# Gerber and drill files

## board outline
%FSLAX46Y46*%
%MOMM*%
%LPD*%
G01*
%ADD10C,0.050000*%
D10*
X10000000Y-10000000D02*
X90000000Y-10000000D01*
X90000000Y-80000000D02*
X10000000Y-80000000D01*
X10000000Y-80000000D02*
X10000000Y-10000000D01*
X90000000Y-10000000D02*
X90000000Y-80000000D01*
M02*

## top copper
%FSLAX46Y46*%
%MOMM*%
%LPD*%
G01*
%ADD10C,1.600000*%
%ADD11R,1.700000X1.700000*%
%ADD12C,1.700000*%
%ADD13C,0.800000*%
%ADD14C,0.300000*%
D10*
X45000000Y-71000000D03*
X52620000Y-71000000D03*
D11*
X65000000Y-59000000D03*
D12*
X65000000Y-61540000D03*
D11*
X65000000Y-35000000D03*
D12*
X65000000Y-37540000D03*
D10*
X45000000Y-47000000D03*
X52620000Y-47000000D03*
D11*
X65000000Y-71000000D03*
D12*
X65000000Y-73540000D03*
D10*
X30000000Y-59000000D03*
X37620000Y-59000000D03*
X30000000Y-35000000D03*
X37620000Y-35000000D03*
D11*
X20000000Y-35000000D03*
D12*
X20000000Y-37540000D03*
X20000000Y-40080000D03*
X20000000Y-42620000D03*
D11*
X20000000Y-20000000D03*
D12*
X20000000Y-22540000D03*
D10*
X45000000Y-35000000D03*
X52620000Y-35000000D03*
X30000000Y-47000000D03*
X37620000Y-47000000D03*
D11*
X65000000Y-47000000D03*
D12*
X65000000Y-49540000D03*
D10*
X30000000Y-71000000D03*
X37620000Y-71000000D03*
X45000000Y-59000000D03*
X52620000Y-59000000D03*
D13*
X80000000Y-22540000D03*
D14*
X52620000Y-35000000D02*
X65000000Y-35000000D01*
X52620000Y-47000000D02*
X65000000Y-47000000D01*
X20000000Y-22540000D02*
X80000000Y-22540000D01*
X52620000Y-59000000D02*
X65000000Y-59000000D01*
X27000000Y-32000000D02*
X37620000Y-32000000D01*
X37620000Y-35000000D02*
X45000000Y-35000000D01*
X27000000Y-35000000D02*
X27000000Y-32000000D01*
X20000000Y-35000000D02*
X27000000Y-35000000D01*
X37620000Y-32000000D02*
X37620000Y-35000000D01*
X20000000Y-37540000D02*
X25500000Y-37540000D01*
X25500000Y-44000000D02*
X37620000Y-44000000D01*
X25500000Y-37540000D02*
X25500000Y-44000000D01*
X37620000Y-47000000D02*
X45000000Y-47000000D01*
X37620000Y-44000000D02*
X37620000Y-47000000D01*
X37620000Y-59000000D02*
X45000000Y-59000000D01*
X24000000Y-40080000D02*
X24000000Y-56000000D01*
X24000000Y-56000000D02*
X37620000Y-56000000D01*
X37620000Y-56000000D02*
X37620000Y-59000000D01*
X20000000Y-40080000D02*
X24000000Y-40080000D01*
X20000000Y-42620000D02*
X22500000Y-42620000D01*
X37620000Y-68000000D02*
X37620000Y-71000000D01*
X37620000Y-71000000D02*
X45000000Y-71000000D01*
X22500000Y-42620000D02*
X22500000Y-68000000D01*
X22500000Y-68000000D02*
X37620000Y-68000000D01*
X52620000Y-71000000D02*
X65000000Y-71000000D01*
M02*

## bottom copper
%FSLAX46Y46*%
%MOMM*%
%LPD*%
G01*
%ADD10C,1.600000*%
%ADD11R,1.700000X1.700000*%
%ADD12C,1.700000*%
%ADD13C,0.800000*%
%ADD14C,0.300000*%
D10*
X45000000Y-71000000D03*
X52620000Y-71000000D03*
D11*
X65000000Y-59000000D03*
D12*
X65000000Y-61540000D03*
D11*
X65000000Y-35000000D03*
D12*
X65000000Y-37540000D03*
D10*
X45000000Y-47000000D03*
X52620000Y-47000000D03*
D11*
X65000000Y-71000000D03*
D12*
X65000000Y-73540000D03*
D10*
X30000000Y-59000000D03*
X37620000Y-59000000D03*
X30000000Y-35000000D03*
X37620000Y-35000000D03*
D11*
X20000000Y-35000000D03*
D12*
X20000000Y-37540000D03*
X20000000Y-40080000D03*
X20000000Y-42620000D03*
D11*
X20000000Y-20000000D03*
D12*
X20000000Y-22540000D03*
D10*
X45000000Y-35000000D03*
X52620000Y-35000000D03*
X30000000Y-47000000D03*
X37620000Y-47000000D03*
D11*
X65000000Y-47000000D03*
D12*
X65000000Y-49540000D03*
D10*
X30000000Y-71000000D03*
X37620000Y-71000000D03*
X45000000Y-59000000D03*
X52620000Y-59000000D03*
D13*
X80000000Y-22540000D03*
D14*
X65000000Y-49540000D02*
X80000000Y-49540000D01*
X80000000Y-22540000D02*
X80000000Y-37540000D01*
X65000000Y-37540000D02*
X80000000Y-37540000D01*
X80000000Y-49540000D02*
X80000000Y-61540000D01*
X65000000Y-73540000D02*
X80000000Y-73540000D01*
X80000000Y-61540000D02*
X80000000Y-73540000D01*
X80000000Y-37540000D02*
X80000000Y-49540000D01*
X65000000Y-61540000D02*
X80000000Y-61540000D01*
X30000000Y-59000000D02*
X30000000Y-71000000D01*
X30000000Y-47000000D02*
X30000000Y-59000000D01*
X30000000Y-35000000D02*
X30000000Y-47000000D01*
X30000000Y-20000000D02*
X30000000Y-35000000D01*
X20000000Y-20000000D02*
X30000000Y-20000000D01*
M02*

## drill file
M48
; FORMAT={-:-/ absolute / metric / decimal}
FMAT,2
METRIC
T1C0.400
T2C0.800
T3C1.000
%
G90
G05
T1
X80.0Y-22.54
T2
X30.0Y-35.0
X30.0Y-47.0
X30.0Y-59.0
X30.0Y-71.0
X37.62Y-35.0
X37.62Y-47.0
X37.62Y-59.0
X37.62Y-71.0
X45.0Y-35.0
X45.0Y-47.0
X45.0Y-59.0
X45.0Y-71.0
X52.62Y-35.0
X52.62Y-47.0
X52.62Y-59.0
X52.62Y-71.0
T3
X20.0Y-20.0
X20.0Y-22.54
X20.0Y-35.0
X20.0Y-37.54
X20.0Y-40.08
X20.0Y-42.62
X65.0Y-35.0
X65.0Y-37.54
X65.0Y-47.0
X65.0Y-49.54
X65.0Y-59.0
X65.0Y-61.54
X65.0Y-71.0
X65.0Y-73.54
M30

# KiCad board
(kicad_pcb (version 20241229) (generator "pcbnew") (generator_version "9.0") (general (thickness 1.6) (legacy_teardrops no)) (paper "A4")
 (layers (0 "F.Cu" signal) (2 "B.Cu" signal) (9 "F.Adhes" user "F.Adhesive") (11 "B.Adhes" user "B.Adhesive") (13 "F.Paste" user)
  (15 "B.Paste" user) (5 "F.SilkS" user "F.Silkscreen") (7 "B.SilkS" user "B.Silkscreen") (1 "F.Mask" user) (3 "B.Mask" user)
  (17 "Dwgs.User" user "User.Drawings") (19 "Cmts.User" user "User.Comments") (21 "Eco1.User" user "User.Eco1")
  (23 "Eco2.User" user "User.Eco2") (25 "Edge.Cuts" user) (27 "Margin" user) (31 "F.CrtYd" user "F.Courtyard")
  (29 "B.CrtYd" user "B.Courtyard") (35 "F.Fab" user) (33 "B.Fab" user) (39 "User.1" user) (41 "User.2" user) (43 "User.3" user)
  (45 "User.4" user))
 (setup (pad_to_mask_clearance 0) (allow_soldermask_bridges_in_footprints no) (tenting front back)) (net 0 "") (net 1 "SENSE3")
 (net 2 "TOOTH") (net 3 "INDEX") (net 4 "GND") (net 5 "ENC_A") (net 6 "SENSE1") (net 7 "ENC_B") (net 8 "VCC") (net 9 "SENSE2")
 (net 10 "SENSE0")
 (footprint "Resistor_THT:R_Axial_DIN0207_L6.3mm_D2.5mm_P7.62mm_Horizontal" (layer "F.Cu") (at 45 71)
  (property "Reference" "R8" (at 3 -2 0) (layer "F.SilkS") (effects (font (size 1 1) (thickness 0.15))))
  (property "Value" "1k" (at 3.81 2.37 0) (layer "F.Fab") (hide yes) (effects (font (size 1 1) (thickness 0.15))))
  (pad "1" thru_hole circle (at 0 0) (size 1.6 1.6) (drill 0.8) (layers "*.Cu" "*.Mask") (remove_unused_layers no) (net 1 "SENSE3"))
  (pad "2" thru_hole circle (at 7.62 0) (size 1.6 1.6) (drill 0.8) (layers "*.Cu" "*.Mask") (remove_unused_layers no) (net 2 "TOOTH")))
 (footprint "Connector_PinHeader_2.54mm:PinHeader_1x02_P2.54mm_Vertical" (layer "F.Cu") (at 65 59)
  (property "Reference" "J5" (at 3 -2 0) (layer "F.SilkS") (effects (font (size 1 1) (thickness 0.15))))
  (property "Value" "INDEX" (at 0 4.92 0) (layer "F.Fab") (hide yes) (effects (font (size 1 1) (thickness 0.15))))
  (pad "1" thru_hole rect (at 0 0) (size 1.7 1.7) (drill 1) (layers "*.Cu" "*.Mask") (remove_unused_layers no) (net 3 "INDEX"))
  (pad "2" thru_hole circle (at 0 2.54) (size 1.7 1.7) (drill 1) (layers "*.Cu" "*.Mask") (remove_unused_layers no) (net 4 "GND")))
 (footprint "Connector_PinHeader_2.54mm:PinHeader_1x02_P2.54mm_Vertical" (layer "F.Cu") (at 65 35)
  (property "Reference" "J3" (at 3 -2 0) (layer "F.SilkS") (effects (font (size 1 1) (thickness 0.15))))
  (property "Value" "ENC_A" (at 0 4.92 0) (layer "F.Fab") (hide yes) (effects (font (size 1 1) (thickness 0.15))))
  (pad "1" thru_hole rect (at 0 0) (size 1.7 1.7) (drill 1) (layers "*.Cu" "*.Mask") (remove_unused_layers no) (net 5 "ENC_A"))
  (pad "2" thru_hole circle (at 0 2.54) (size 1.7 1.7) (drill 1) (layers "*.Cu" "*.Mask") (remove_unused_layers no) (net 4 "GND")))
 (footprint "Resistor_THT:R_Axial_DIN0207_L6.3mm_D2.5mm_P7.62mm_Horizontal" (layer "F.Cu") (at 45 47)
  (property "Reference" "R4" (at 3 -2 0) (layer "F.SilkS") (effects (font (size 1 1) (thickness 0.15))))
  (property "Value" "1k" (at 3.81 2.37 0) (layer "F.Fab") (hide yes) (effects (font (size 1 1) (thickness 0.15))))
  (pad "1" thru_hole circle (at 0 0) (size 1.6 1.6) (drill 0.8) (layers "*.Cu" "*.Mask") (remove_unused_layers no) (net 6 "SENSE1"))
  (pad "2" thru_hole circle (at 7.62 0) (size 1.6 1.6) (drill 0.8) (layers "*.Cu" "*.Mask") (remove_unused_layers no) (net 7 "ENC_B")))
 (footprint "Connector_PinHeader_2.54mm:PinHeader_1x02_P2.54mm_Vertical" (layer "F.Cu") (at 65 71)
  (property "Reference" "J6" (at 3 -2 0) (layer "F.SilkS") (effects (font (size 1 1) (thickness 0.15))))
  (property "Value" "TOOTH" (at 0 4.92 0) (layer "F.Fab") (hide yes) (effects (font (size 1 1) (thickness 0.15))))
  (pad "1" thru_hole rect (at 0 0) (size 1.7 1.7) (drill 1) (layers "*.Cu" "*.Mask") (remove_unused_layers no) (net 2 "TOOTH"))
  (pad "2" thru_hole circle (at 0 2.54) (size 1.7 1.7) (drill 1) (layers "*.Cu" "*.Mask") (remove_unused_layers no) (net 4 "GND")))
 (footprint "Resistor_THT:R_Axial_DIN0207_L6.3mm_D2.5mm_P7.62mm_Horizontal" (layer "F.Cu") (at 30 59)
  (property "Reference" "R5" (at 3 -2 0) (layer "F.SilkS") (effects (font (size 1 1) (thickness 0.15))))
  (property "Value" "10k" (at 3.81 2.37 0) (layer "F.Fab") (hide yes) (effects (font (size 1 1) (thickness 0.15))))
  (pad "1" thru_hole circle (at 0 0) (size 1.6 1.6) (drill 0.8) (layers "*.Cu" "*.Mask") (remove_unused_layers no) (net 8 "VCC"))
  (pad "2" thru_hole circle (at 7.62 0) (size 1.6 1.6) (drill 0.8) (layers "*.Cu" "*.Mask") (remove_unused_layers no) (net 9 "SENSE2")))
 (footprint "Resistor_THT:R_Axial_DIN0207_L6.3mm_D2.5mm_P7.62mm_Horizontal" (layer "F.Cu") (at 30 35)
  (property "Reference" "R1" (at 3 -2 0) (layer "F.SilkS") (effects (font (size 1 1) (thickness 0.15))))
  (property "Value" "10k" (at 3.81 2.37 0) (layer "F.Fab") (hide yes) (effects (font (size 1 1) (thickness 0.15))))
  (pad "1" thru_hole circle (at 0 0) (size 1.6 1.6) (drill 0.8) (layers "*.Cu" "*.Mask") (remove_unused_layers no) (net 8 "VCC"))
  (pad "2" thru_hole circle (at 7.62 0) (size 1.6 1.6) (drill 0.8) (layers "*.Cu" "*.Mask") (remove_unused_layers no) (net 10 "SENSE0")))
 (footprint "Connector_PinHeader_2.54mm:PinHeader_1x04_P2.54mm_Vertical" (layer "F.Cu") (at 20 35)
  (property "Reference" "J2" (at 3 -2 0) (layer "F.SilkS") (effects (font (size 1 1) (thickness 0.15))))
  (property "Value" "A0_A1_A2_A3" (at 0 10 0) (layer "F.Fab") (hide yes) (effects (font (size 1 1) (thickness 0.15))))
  (pad "1" thru_hole rect (at 0 0) (size 1.7 1.7) (drill 1) (layers "*.Cu" "*.Mask") (remove_unused_layers no) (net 10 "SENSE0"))
  (pad "2" thru_hole circle (at 0 2.54) (size 1.7 1.7) (drill 1) (layers "*.Cu" "*.Mask") (remove_unused_layers no) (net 6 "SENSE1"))
  (pad "3" thru_hole circle (at 0 5.08) (size 1.7 1.7) (drill 1) (layers "*.Cu" "*.Mask") (remove_unused_layers no) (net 9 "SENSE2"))
  (pad "4" thru_hole circle (at 0 7.62) (size 1.7 1.7) (drill 1) (layers "*.Cu" "*.Mask") (remove_unused_layers no) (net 1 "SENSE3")))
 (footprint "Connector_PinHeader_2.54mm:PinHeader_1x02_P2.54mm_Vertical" (layer "F.Cu") (at 20 20)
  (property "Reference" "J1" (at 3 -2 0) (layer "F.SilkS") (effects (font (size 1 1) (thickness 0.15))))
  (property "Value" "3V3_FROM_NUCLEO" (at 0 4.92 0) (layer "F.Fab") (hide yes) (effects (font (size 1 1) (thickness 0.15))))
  (pad "1" thru_hole rect (at 0 0) (size 1.7 1.7) (drill 1) (layers "*.Cu" "*.Mask") (remove_unused_layers no) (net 8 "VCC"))
  (pad "2" thru_hole circle (at 0 2.54) (size 1.7 1.7) (drill 1) (layers "*.Cu" "*.Mask") (remove_unused_layers no) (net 4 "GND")))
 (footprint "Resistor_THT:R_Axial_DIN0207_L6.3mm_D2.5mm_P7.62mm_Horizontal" (layer "F.Cu") (at 45 35)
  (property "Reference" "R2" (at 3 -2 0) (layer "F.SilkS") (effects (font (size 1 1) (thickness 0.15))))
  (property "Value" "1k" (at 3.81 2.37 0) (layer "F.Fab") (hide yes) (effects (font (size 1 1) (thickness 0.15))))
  (pad "1" thru_hole circle (at 0 0) (size 1.6 1.6) (drill 0.8) (layers "*.Cu" "*.Mask") (remove_unused_layers no) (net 10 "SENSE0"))
  (pad "2" thru_hole circle (at 7.62 0) (size 1.6 1.6) (drill 0.8) (layers "*.Cu" "*.Mask") (remove_unused_layers no) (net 5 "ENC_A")))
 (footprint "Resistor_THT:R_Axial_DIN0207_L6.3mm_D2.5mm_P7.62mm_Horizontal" (layer "F.Cu") (at 30 47)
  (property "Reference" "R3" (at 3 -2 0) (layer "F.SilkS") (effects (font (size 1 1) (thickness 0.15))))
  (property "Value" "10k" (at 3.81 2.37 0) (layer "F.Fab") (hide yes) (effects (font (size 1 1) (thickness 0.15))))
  (pad "1" thru_hole circle (at 0 0) (size 1.6 1.6) (drill 0.8) (layers "*.Cu" "*.Mask") (remove_unused_layers no) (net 8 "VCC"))
  (pad "2" thru_hole circle (at 7.62 0) (size 1.6 1.6) (drill 0.8) (layers "*.Cu" "*.Mask") (remove_unused_layers no) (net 6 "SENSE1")))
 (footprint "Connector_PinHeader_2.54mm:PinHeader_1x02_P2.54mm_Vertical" (layer "F.Cu") (at 65 47)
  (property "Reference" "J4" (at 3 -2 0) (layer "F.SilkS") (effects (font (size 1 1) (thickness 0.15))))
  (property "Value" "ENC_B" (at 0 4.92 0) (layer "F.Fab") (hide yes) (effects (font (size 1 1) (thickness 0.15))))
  (pad "1" thru_hole rect (at 0 0) (size 1.7 1.7) (drill 1) (layers "*.Cu" "*.Mask") (remove_unused_layers no) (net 7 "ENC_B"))
  (pad "2" thru_hole circle (at 0 2.54) (size 1.7 1.7) (drill 1) (layers "*.Cu" "*.Mask") (remove_unused_layers no) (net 4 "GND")))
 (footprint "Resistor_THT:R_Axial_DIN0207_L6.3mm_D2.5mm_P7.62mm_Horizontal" (layer "F.Cu") (at 30 71)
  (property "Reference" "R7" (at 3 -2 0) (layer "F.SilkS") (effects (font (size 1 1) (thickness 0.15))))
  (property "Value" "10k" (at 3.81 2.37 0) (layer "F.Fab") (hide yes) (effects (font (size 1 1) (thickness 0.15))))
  (pad "1" thru_hole circle (at 0 0) (size 1.6 1.6) (drill 0.8) (layers "*.Cu" "*.Mask") (remove_unused_layers no) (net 8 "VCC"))
  (pad "2" thru_hole circle (at 7.62 0) (size 1.6 1.6) (drill 0.8) (layers "*.Cu" "*.Mask") (remove_unused_layers no) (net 1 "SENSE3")))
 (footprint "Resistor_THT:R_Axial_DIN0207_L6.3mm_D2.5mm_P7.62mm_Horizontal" (layer "F.Cu") (at 45 59)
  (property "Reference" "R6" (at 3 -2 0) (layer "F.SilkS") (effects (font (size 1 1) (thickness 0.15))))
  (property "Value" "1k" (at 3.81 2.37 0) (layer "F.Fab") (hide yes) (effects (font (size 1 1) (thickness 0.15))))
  (pad "1" thru_hole circle (at 0 0) (size 1.6 1.6) (drill 0.8) (layers "*.Cu" "*.Mask") (remove_unused_layers no) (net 9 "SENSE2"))
  (pad "2" thru_hole circle (at 7.62 0) (size 1.6 1.6) (drill 0.8) (layers "*.Cu" "*.Mask") (remove_unused_layers no) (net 3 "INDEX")))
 (gr_line (start 10 10) (end 90 10) (stroke (width 0.05) (type default)) (layer "Edge.Cuts"))
 (gr_line (start 90 80) (end 10 80) (stroke (width 0.05) (type default)) (layer "Edge.Cuts"))
 (gr_line (start 10 80) (end 10 10) (stroke (width 0.05) (type default)) (layer "Edge.Cuts"))
 (gr_line (start 90 10) (end 90 80) (stroke (width 0.05) (type default)) (layer "Edge.Cuts"))
 (segment (start 52.62 35) (end 65 35) (width 0.3) (layer "F.Cu") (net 5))
 (segment (start 52.62 47) (end 65 47) (width 0.3) (layer "F.Cu") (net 7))
 (segment (start 20 22.54) (end 80 22.54) (width 0.3) (layer "F.Cu") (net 4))
 (via (at 80 22.54) (size 0.8) (drill 0.4) (layers "F.Cu" "B.Cu") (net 4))
 (segment (start 65 49.54) (end 80 49.54) (width 0.3) (layer "B.Cu") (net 4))
 (segment (start 80 22.54) (end 80 37.54) (width 0.3) (layer "B.Cu") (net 4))
 (segment (start 65 37.54) (end 80 37.54) (width 0.3) (layer "B.Cu") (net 4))
 (segment (start 80 49.54) (end 80 61.54) (width 0.3) (layer "B.Cu") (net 4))
 (segment (start 65 73.54) (end 80 73.54) (width 0.3) (layer "B.Cu") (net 4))
 (segment (start 80 61.54) (end 80 73.54) (width 0.3) (layer "B.Cu") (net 4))
 (segment (start 80 37.54) (end 80 49.54) (width 0.3) (layer "B.Cu") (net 4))
 (segment (start 65 61.54) (end 80 61.54) (width 0.3) (layer "B.Cu") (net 4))
 (segment (start 52.62 59) (end 65 59) (width 0.3) (layer "F.Cu") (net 3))
 (segment (start 27 32) (end 37.62 32) (width 0.3) (layer "F.Cu") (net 10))
 (segment (start 37.62 35) (end 45 35) (width 0.3) (layer "F.Cu") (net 10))
 (segment (start 27 35) (end 27 32) (width 0.3) (layer "F.Cu") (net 10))
 (segment (start 20 35) (end 27 35) (width 0.3) (layer "F.Cu") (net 10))
 (segment (start 37.62 32) (end 37.62 35) (width 0.3) (layer "F.Cu") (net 10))
 (segment (start 20 37.54) (end 25.5 37.54) (width 0.3) (layer "F.Cu") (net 6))
 (segment (start 25.5 44) (end 37.62 44) (width 0.3) (layer "F.Cu") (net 6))
 (segment (start 25.5 37.54) (end 25.5 44) (width 0.3) (layer "F.Cu") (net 6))
 (segment (start 37.62 47) (end 45 47) (width 0.3) (layer "F.Cu") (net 6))
 (segment (start 37.62 44) (end 37.62 47) (width 0.3) (layer "F.Cu") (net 6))
 (segment (start 37.62 59) (end 45 59) (width 0.3) (layer "F.Cu") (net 9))
 (segment (start 24 40.08) (end 24 56) (width 0.3) (layer "F.Cu") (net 9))
 (segment (start 24 56) (end 37.62 56) (width 0.3) (layer "F.Cu") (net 9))
 (segment (start 37.62 56) (end 37.62 59) (width 0.3) (layer "F.Cu") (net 9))
 (segment (start 20 40.08) (end 24 40.08) (width 0.3) (layer "F.Cu") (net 9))
 (segment (start 20 42.62) (end 22.5 42.62) (width 0.3) (layer "F.Cu") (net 1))
 (segment (start 37.62 68) (end 37.62 71) (width 0.3) (layer "F.Cu") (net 1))
 (segment (start 37.62 71) (end 45 71) (width 0.3) (layer "F.Cu") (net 1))
 (segment (start 22.5 42.62) (end 22.5 68) (width 0.3) (layer "F.Cu") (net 1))
 (segment (start 22.5 68) (end 37.62 68) (width 0.3) (layer "F.Cu") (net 1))
 (segment (start 52.62 71) (end 65 71) (width 0.3) (layer "F.Cu") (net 2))
 (segment (start 30 59) (end 30 71) (width 0.3) (layer "B.Cu") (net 8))
 (segment (start 30 47) (end 30 59) (width 0.3) (layer "B.Cu") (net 8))
 (segment (start 30 35) (end 30 47) (width 0.3) (layer "B.Cu") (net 8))
 (segment (start 30 20) (end 30 35) (width 0.3) (layer "B.Cu") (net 8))
 (segment (start 20 20) (end 30 20) (width 0.3) (layer "B.Cu") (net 8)))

